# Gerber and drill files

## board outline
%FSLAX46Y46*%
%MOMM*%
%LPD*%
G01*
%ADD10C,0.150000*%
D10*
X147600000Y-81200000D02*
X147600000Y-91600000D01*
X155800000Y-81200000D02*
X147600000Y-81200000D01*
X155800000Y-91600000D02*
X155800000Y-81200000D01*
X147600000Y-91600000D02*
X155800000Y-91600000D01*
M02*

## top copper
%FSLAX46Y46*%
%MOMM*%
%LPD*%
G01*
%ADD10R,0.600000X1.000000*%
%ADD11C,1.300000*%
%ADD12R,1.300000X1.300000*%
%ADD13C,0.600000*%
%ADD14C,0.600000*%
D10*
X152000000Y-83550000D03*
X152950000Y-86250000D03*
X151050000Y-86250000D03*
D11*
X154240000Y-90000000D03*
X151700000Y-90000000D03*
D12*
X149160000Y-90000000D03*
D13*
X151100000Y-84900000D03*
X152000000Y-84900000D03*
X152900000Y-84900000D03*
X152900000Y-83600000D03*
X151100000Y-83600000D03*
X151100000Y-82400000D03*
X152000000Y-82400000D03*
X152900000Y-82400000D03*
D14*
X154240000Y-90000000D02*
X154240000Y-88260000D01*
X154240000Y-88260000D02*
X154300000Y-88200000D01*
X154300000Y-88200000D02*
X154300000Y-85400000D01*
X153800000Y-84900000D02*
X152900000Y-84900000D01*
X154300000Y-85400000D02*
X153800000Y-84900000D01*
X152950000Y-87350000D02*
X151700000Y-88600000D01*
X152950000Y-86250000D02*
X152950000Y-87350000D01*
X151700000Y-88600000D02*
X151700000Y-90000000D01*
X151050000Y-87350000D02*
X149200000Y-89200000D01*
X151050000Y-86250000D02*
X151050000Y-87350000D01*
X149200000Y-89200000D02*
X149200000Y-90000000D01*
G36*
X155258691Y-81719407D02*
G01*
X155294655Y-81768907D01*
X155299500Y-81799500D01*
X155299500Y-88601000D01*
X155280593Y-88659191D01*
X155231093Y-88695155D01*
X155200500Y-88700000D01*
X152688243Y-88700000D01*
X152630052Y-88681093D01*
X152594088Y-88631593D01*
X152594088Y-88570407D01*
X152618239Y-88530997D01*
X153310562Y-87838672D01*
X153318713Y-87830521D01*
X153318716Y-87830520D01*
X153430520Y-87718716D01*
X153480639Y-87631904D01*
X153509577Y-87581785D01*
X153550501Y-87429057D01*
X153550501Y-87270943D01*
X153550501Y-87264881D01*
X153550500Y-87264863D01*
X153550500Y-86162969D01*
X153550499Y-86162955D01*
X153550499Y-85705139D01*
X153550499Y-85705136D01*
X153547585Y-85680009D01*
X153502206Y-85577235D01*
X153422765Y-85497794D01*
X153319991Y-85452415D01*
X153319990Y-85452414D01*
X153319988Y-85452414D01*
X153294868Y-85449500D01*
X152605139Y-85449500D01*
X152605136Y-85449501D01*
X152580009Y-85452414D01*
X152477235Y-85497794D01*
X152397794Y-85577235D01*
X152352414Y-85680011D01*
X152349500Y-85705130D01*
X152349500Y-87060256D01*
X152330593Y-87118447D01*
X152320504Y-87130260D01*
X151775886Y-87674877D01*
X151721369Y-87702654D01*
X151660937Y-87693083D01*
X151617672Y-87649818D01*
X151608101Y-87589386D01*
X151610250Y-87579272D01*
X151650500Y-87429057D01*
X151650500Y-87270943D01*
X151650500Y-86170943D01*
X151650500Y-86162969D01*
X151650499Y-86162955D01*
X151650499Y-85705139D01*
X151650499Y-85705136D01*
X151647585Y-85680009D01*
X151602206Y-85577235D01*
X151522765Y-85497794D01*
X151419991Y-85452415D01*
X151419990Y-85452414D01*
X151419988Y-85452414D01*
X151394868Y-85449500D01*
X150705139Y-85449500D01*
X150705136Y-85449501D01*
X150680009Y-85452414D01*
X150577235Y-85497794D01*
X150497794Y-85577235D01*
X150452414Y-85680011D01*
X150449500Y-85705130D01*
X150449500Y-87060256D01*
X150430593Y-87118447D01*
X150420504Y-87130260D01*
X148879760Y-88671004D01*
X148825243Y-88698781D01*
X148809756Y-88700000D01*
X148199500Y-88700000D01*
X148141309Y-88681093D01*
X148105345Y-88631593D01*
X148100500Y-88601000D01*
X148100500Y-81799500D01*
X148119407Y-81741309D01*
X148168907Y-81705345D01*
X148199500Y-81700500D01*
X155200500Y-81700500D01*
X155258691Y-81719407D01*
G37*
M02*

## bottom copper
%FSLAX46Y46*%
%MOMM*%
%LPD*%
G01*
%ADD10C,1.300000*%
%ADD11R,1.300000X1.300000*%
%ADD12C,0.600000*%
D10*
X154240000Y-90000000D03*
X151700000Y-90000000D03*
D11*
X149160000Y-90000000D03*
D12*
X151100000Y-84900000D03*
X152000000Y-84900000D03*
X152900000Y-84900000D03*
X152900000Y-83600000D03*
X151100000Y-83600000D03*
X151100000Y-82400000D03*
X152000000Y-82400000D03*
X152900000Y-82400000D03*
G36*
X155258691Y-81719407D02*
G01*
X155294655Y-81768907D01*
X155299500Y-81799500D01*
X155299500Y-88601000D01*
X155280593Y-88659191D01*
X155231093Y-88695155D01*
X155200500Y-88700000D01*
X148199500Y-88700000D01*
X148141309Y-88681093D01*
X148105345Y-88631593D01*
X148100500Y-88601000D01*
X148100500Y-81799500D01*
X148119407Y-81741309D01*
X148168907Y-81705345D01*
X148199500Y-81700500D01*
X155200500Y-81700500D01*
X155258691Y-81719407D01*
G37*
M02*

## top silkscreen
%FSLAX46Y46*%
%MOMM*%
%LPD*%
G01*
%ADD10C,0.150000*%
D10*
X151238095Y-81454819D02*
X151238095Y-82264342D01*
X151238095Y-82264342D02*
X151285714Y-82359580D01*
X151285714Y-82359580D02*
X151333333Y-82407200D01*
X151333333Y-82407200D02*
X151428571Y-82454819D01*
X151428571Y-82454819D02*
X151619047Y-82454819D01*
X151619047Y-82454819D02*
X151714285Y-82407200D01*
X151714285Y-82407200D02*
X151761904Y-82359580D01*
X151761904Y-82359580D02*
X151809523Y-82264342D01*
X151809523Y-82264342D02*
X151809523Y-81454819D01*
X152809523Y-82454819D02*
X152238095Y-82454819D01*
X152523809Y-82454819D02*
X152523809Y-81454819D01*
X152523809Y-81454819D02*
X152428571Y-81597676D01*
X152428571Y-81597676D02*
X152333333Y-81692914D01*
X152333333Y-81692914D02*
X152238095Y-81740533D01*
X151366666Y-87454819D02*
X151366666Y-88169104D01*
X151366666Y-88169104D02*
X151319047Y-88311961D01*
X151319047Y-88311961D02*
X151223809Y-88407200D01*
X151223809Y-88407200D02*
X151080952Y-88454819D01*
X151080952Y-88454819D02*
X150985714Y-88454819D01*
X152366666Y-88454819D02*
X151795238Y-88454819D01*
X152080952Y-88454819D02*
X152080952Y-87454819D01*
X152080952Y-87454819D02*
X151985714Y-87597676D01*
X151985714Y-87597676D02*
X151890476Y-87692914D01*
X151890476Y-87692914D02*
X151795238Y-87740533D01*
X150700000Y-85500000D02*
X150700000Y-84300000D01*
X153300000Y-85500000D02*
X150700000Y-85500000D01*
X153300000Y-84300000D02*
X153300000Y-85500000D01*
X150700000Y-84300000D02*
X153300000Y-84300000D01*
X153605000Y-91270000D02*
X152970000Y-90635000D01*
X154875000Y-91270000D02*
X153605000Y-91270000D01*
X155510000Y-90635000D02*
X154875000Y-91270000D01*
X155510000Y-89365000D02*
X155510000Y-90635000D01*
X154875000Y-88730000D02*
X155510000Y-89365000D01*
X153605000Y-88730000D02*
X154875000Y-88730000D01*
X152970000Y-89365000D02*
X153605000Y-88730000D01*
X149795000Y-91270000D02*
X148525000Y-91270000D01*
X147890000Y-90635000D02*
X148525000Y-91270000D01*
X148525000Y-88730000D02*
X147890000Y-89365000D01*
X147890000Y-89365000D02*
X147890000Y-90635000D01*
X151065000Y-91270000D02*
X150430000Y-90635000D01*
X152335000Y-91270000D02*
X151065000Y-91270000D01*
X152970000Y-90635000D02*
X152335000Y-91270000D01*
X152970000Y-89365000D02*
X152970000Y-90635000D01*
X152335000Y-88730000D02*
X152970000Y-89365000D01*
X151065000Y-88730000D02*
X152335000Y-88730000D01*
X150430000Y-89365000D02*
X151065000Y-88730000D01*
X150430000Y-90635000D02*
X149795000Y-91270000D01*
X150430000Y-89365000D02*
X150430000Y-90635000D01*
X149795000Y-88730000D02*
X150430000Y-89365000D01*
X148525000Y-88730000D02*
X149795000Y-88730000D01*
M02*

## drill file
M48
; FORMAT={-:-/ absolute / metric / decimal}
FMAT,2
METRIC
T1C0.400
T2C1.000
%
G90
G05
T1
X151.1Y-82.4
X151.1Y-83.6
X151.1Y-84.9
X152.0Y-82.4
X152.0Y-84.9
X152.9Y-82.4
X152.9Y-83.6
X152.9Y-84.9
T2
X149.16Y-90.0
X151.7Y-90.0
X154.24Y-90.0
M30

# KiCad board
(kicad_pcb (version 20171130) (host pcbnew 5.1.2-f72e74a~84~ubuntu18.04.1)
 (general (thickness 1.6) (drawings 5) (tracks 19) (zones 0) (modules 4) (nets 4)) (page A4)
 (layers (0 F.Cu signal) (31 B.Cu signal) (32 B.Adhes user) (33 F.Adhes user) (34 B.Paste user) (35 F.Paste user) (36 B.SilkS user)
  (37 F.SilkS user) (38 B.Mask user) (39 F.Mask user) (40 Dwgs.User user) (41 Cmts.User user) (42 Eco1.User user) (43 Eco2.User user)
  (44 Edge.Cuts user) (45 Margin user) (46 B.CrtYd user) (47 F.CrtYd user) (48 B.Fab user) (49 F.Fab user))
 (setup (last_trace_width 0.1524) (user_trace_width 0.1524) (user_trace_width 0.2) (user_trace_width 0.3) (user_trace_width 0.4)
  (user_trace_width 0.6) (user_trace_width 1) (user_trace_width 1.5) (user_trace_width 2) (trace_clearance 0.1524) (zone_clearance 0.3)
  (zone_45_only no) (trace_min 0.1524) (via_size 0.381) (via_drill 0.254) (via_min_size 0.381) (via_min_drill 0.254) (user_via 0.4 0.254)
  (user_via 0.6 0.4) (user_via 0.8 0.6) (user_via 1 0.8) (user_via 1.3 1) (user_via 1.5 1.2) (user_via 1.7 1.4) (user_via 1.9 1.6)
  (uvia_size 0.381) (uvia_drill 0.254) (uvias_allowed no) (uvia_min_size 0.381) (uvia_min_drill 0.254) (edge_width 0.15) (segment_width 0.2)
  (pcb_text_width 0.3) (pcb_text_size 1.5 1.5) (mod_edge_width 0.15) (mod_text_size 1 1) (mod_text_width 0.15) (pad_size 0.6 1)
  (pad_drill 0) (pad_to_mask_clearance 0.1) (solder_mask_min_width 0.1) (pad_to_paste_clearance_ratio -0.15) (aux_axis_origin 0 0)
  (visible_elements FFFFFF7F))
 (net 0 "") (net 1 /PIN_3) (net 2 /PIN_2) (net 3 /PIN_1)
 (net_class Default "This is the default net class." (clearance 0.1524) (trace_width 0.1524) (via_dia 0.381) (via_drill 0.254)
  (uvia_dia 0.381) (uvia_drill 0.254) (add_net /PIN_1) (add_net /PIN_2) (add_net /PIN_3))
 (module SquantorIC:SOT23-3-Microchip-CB (layer F.Cu) (at 152 84.9)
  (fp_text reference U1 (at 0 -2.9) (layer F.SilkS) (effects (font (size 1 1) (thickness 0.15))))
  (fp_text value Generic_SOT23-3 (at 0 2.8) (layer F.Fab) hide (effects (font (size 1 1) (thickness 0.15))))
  (fp_line (start -1.3 0.6) (end -1.3 -0.6) (layer F.SilkS) (width 0.15))
  (fp_line (start 1.3 0.6) (end -1.3 0.6) (layer F.SilkS) (width 0.15))
  (fp_line (start 1.3 -0.6) (end 1.3 0.6) (layer F.SilkS) (width 0.15))
  (fp_line (start -1.3 -0.6) (end 1.3 -0.6) (layer F.SilkS) (width 0.15))
  (pad 3 smd rect (at 0 -1.35) (size 0.6 1) (layers F.Cu F.Paste F.Mask) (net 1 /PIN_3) (zone_connect 2))
  (pad 2 smd rect (at 0.95 1.35) (size 0.6 1) (layers F.Cu F.Paste F.Mask) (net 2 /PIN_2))
  (pad 1 smd rect (at -0.95 1.35) (size 0.6 1) (layers F.Cu F.Paste F.Mask) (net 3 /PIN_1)))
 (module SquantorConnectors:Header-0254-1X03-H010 (layer F.Cu) (at 151.7 90)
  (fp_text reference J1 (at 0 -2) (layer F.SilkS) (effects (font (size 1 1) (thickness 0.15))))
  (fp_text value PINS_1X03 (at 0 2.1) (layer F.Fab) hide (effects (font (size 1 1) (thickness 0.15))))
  (fp_line (start 1.905 1.27) (end 1.27 0.635) (layer F.SilkS) (width 0.15))
  (fp_line (start 3.175 1.27) (end 1.905 1.27) (layer F.SilkS) (width 0.15))
  (fp_line (start 3.81 0.635) (end 3.175 1.27) (layer F.SilkS) (width 0.15))
  (fp_line (start 3.81 -0.635) (end 3.81 0.635) (layer F.SilkS) (width 0.15))
  (fp_line (start 3.175 -1.27) (end 3.81 -0.635) (layer F.SilkS) (width 0.15))
  (fp_line (start 1.905 -1.27) (end 3.175 -1.27) (layer F.SilkS) (width 0.15))
  (fp_line (start 1.27 -0.635) (end 1.905 -1.27) (layer F.SilkS) (width 0.15))
  (fp_line (start -1.905 1.27) (end -3.175 1.27) (layer F.SilkS) (width 0.15))
  (fp_line (start -3.81 0.635) (end -3.175 1.27) (layer F.SilkS) (width 0.15))
  (fp_line (start -3.175 -1.27) (end -3.81 -0.635) (layer F.SilkS) (width 0.15))
  (fp_line (start -3.81 -0.635) (end -3.81 0.635) (layer F.SilkS) (width 0.15))
  (fp_line (start -0.635 1.27) (end -1.27 0.635) (layer F.SilkS) (width 0.15))
  (fp_line (start 0.635 1.27) (end -0.635 1.27) (layer F.SilkS) (width 0.15))
  (fp_line (start 1.27 0.635) (end 0.635 1.27) (layer F.SilkS) (width 0.15))
  (fp_line (start 1.27 -0.635) (end 1.27 0.635) (layer F.SilkS) (width 0.15))
  (fp_line (start 0.635 -1.27) (end 1.27 -0.635) (layer F.SilkS) (width 0.15))
  (fp_line (start -0.635 -1.27) (end 0.635 -1.27) (layer F.SilkS) (width 0.15))
  (fp_line (start -1.27 -0.635) (end -0.635 -1.27) (layer F.SilkS) (width 0.15))
  (fp_line (start -1.27 0.635) (end -1.905 1.27) (layer F.SilkS) (width 0.15))
  (fp_line (start -1.27 -0.635) (end -1.27 0.635) (layer F.SilkS) (width 0.15))
  (fp_line (start -1.905 -1.27) (end -1.27 -0.635) (layer F.SilkS) (width 0.15))
  (fp_line (start -3.175 -1.27) (end -1.905 -1.27) (layer F.SilkS) (width 0.15))
  (pad 3 thru_hole circle (at 2.54 0 180) (size 1.3 1.3) (drill 1) (layers *.Cu *.Mask) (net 1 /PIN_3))
  (pad 2 thru_hole circle (at 0 0 180) (size 1.3 1.3) (drill 1) (layers *.Cu *.Mask) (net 2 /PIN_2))
  (pad 1 thru_hole rect (at -2.54 0 180) (size 1.3 1.3) (drill 1) (layers *.Cu *.Mask) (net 3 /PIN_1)))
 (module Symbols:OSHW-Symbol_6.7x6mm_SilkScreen (layer B.Cu) (at 152 84.6 180)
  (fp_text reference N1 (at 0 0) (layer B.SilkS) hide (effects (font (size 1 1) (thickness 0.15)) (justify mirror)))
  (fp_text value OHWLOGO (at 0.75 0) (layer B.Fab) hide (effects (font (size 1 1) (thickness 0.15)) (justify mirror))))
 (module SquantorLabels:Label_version (layer B.Cu) (at 152 88.2)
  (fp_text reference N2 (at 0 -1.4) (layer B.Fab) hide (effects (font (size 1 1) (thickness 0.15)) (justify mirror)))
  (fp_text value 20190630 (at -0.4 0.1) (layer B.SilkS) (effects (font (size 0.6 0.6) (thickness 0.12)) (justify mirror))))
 (gr_line (start 147.6 81.2) (end 147.6 91.6) (layer Edge.Cuts) (width 0.15))
 (gr_line (start 155.8 81.2) (end 147.6 81.2) (layer Edge.Cuts) (width 0.15))
 (gr_line (start 155.8 91.6) (end 155.8 81.2) (layer Edge.Cuts) (width 0.15))
 (gr_line (start 147.6 91.6) (end 155.8 91.6) (layer Edge.Cuts) (width 0.15))
 (via (at 151.1 84.9) (size 0.6) (drill 0.4) (layers F.Cu B.Cu) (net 1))
 (via (at 152 84.9) (size 0.6) (drill 0.4) (layers F.Cu B.Cu) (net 1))
 (via (at 152.9 84.9) (size 0.6) (drill 0.4) (layers F.Cu B.Cu) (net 1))
 (via (at 152.9 83.6) (size 0.6) (drill 0.4) (layers F.Cu B.Cu) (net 1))
 (via (at 151.1 83.6) (size 0.6) (drill 0.4) (layers F.Cu B.Cu) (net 1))
 (via (at 151.1 82.4) (size 0.6) (drill 0.4) (layers F.Cu B.Cu) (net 1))
 (via (at 152 82.4) (size 0.6) (drill 0.4) (layers F.Cu B.Cu) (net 1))
 (via (at 152.9 82.4) (size 0.6) (drill 0.4) (layers F.Cu B.Cu) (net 1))
 (segment (start 154.24 90) (end 154.24 88.26) (width 0.6) (layer F.Cu) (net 1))
 (segment (start 154.24 88.26) (end 154.3 88.2) (width 0.6) (layer F.Cu) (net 1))
 (segment (start 154.3 88.2) (end 154.3 85.4) (width 0.6) (layer F.Cu) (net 1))
 (segment (start 153.8 84.9) (end 152.9 84.9) (width 0.6) (layer F.Cu) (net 1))
 (segment (start 154.3 85.4) (end 153.8 84.9) (width 0.6) (layer F.Cu) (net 1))
 (segment (start 152.95 87.35) (end 151.7 88.6) (width 0.6) (layer F.Cu) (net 2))
 (segment (start 152.95 86.25) (end 152.95 87.35) (width 0.6) (layer F.Cu) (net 2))
 (segment (start 151.7 88.6) (end 151.7 90) (width 0.6) (layer F.Cu) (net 2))
 (segment (start 151.05 87.35) (end 149.2 89.2) (width 0.6) (layer F.Cu) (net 3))
 (segment (start 151.05 86.25) (end 151.05 87.35) (width 0.6) (layer F.Cu) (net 3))
 (segment (start 149.2 89.2) (end 149.2 90) (width 0.6) (layer F.Cu) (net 3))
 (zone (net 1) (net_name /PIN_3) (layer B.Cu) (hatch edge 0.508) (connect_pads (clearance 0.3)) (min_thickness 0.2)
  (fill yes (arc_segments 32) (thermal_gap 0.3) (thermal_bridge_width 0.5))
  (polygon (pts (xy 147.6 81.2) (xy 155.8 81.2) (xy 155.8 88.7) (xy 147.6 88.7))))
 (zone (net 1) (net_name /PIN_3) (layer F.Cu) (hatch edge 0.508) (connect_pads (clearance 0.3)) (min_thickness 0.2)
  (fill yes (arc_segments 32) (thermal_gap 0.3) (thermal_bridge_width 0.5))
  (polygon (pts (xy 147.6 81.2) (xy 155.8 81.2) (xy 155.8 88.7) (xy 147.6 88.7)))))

